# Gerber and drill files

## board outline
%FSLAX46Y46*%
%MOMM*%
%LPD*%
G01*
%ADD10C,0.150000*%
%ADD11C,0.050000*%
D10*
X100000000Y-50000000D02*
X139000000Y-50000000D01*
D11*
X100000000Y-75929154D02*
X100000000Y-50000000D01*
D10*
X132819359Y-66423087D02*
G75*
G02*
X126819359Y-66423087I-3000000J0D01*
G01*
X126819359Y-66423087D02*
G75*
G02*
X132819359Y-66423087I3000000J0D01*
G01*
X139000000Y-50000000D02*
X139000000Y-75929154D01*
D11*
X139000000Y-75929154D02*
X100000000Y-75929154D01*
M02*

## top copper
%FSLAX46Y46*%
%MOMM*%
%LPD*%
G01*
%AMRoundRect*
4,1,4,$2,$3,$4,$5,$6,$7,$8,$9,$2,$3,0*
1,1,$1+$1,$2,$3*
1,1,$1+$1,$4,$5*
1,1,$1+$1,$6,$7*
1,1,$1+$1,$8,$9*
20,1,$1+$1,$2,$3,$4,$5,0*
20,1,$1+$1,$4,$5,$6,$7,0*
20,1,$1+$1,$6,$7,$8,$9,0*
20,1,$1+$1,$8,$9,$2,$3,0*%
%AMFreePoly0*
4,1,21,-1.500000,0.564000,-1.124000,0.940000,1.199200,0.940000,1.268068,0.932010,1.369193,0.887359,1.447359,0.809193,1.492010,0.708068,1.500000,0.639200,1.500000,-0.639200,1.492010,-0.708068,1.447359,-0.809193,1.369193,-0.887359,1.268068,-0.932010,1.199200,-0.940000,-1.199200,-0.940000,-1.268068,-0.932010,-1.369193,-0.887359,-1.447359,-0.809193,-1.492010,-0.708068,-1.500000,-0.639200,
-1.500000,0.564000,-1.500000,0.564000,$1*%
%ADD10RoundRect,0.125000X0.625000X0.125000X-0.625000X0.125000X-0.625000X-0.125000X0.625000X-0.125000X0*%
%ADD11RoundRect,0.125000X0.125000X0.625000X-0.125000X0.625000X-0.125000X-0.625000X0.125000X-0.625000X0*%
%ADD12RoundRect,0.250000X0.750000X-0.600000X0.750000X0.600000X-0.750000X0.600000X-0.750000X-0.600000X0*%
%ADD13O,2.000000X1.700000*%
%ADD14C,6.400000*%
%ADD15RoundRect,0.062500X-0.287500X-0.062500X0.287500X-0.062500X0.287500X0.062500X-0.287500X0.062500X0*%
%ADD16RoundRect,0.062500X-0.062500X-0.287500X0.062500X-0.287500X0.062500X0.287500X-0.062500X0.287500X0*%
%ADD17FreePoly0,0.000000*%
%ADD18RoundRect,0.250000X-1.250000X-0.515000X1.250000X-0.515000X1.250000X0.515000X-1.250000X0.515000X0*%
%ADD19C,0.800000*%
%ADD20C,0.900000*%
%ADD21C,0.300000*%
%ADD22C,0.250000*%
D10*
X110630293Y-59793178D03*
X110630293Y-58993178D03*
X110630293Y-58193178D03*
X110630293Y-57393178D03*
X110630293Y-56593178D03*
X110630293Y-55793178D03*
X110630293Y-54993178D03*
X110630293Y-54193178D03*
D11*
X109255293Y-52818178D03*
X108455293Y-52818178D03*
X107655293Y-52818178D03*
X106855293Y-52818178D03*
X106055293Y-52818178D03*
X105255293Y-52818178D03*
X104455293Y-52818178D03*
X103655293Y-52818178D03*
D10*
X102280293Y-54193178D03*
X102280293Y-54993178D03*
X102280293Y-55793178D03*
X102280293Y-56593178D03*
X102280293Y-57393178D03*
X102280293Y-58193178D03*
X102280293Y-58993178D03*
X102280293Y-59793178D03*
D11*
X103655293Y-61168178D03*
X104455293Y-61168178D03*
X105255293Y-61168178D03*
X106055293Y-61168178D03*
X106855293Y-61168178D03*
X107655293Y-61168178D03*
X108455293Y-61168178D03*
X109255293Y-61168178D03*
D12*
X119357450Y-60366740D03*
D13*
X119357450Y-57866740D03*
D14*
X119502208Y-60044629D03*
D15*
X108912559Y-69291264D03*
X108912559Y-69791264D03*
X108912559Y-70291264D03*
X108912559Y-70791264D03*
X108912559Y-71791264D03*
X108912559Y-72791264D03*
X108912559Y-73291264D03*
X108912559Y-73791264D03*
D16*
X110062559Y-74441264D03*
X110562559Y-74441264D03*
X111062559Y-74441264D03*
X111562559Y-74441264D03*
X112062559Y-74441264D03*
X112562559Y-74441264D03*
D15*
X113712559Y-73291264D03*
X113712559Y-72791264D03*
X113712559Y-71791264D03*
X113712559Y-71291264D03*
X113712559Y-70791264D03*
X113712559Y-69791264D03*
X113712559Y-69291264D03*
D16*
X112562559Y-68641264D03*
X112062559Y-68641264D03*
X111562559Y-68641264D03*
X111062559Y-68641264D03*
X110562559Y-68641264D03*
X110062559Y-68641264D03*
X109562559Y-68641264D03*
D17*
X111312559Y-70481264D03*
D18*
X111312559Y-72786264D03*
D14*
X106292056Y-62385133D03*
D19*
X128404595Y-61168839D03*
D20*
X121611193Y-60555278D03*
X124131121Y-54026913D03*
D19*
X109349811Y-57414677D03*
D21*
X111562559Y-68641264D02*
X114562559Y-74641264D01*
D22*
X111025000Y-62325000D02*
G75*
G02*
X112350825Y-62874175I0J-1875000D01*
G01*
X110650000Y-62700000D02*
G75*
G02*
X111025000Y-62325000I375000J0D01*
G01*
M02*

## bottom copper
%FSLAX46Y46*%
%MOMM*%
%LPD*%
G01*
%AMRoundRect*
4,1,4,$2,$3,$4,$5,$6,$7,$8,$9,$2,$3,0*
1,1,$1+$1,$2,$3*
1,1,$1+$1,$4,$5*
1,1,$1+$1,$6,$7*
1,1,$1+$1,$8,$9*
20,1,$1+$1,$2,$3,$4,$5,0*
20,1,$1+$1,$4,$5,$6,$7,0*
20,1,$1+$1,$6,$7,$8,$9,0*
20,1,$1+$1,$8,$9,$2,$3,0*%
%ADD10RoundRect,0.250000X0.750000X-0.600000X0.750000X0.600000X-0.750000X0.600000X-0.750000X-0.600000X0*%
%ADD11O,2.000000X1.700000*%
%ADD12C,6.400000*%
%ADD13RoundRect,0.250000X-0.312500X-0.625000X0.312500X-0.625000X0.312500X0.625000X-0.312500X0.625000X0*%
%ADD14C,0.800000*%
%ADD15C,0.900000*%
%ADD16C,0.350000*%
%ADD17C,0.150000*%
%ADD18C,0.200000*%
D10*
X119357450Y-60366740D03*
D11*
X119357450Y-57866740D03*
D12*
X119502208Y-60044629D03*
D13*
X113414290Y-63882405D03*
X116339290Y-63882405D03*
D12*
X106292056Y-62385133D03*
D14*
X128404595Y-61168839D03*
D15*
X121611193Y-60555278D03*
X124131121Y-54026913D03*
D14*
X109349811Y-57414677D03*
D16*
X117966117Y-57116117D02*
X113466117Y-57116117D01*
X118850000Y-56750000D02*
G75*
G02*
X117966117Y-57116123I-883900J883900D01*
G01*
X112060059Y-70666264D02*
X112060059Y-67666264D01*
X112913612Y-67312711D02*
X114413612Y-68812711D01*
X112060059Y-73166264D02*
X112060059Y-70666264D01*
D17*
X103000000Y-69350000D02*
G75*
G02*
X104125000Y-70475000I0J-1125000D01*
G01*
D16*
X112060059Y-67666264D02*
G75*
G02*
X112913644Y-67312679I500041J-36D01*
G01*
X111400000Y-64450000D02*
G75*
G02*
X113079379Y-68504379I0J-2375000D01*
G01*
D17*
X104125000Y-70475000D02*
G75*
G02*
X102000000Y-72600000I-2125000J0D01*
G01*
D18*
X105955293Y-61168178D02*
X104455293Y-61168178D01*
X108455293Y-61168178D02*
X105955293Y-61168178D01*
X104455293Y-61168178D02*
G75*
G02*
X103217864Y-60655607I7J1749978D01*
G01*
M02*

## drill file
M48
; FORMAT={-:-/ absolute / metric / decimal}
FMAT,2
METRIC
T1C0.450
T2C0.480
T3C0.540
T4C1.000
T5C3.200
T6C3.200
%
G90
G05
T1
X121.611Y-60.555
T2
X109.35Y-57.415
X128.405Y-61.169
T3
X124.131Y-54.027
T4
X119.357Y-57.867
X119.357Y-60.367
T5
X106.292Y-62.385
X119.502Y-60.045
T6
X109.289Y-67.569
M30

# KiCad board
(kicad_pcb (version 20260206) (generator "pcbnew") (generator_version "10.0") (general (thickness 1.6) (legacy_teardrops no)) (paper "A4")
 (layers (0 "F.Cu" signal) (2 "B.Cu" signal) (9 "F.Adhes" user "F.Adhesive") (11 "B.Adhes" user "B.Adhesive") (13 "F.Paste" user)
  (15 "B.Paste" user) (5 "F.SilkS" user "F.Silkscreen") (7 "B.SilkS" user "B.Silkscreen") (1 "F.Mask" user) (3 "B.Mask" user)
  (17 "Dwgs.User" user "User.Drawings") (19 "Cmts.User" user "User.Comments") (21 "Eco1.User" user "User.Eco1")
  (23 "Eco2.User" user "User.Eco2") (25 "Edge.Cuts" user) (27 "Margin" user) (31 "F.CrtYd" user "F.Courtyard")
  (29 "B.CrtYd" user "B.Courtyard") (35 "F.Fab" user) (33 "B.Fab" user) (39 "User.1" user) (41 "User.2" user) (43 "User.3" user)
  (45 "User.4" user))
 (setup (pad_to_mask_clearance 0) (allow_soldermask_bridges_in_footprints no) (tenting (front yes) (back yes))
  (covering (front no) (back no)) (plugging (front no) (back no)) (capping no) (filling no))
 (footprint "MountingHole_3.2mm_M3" (layer "F.Cu") (at 109.289246 67.568769)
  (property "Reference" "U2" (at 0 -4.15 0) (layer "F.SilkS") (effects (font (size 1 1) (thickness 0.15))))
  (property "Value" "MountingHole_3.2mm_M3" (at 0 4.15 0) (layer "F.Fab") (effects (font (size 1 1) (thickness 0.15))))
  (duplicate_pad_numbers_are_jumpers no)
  (pad "" np_thru_hole circle (at 0 0) (size 3.2 3.2) (drill 3.2) (layers "*.Cu" "*.Mask")))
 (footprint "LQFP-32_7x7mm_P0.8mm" (layer "F.Cu") (at 106.455293 56.993178 180)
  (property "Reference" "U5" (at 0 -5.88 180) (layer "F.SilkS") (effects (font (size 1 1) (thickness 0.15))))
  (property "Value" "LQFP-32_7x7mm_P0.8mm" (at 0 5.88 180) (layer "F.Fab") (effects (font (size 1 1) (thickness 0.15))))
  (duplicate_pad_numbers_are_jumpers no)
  (pad "1" smd roundrect (at -4.175 -2.8 180) (size 1.5 0.5) (layers "F.Cu" "F.Mask" "F.Paste") (roundrect_rratio 0.25) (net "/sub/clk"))
  (pad "2" smd roundrect (at -4.175 -2 180) (size 1.5 0.5) (layers "F.Cu" "F.Mask" "F.Paste") (roundrect_rratio 0.25) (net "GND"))
  (pad "3" smd roundrect (at -4.175 -1.2 180) (size 1.5 0.5) (layers "F.Cu" "F.Mask" "F.Paste") (roundrect_rratio 0.25) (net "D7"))
  (pad "4" smd roundrect (at -4.175 -0.4 180) (size 1.5 0.5) (layers "F.Cu" "F.Mask" "F.Paste") (roundrect_rratio 0.25) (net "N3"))
  (pad "5" smd roundrect (at -4.175 0.4 180) (size 1.5 0.5) (layers "F.Cu" "F.Mask" "F.Paste") (roundrect_rratio 0.25))
  (pad "6" smd roundrect (at -4.175 1.2 180) (size 1.5 0.5) (layers "F.Cu" "F.Mask" "F.Paste") (roundrect_rratio 0.25) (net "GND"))
  (pad "7" smd roundrect (at -4.175 2 180) (size 1.5 0.5) (layers "F.Cu" "F.Mask" "F.Paste") (roundrect_rratio 0.25))
  (pad "8" smd roundrect (at -4.175 2.8 180) (size 1.5 0.5) (layers "F.Cu" "F.Mask" "F.Paste") (roundrect_rratio 0.25) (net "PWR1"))
  (pad "9" smd roundrect (at -2.8 4.175 180) (size 0.5 1.5) (layers "F.Cu" "F.Mask" "F.Paste") (roundrect_rratio 0.25) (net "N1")
   (clearance 0.35))
  (pad "10" smd roundrect (at -2 4.175 180) (size 0.5 1.5) (layers "F.Cu" "F.Mask" "F.Paste") (roundrect_rratio 0.25) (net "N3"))
  (pad "11" smd roundrect (at -1.2 4.175 180) (size 0.5 1.5) (layers "F.Cu" "F.Mask" "F.Paste") (roundrect_rratio 0.25) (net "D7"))
  (pad "12" smd roundrect (at -0.4 4.175 180) (size 0.5 1.5) (layers "F.Cu" "F.Mask" "F.Paste") (roundrect_rratio 0.25) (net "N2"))
  (pad "13" smd roundrect (at 0.4 4.175 180) (size 0.5 1.5) (layers "F.Cu" "F.Mask" "F.Paste") (roundrect_rratio 0.25) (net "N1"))
  (pad "14" smd roundrect (at 1.2 4.175 180) (size 0.5 1.5) (layers "F.Cu" "F.Mask" "F.Paste") (roundrect_rratio 0.25) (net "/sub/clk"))
  (pad "15" smd roundrect (at 2 4.175 180) (size 0.5 1.5) (layers "F.Cu" "F.Mask" "F.Paste") (roundrect_rratio 0.25))
  (pad "16" smd roundrect (at 2.8 4.175 180) (size 0.5 1.5) (layers "F.Cu" "F.Mask" "F.Paste") (roundrect_rratio 0.25))
  (pad "17" smd roundrect (at 4.175 2.8 180) (size 1.5 0.5) (layers "F.Cu" "F.Mask" "F.Paste") (roundrect_rratio 0.25) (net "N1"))
  (pad "18" smd roundrect (at 4.175 2 180) (size 1.5 0.5) (layers "F.Cu" "F.Mask" "F.Paste") (roundrect_rratio 0.25) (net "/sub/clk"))
  (pad "19" smd roundrect (at 4.175 1.2 180) (size 1.5 0.5) (layers "F.Cu" "F.Mask" "F.Paste") (roundrect_rratio 0.25) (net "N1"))
  (pad "20" smd roundrect (at 4.175 0.4 180) (size 1.5 0.5) (layers "F.Cu" "F.Mask" "F.Paste") (roundrect_rratio 0.25) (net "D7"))
  (pad "21" smd roundrect (at 4.175 -0.4 180) (size 1.5 0.5) (layers "F.Cu" "F.Mask" "F.Paste") (roundrect_rratio 0.25) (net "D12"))
  (pad "22" smd roundrect (at 4.175 -1.2 180) (size 1.5 0.5) (layers "F.Cu" "F.Mask" "F.Paste") (roundrect_rratio 0.25))
  (pad "23" smd roundrect (at 4.175 -2 180) (size 1.5 0.5) (layers "F.Cu" "F.Mask" "F.Paste") (roundrect_rratio 0.25))
  (pad "24" smd roundrect (at 4.175 -2.8 180) (size 1.5 0.5) (layers "F.Cu" "F.Mask" "F.Paste") (roundrect_rratio 0.25))
  (pad "25" smd roundrect (at 2.8 -4.175 180) (size 0.5 1.5) (layers "F.Cu" "F.Mask" "F.Paste") (roundrect_rratio 0.25) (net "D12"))
  (pad "26" smd roundrect (at 2 -4.175 180) (size 0.5 1.5) (layers "F.Cu" "F.Mask" "F.Paste") (roundrect_rratio 0.25) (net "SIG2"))
  (pad "27" smd roundrect (at 1.2 -4.175 180) (size 0.5 1.5) (layers "F.Cu" "F.Mask" "F.Paste") (roundrect_rratio 0.25) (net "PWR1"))
  (pad "28" smd roundrect (at 0.4 -4.175 180) (size 0.5 1.5) (layers "F.Cu" "F.Mask" "F.Paste") (roundrect_rratio 0.25) (clearance 0.35))
  (pad "29" smd roundrect (at -0.4 -4.175 180) (size 0.5 1.5) (layers "F.Cu" "F.Mask" "F.Paste") (roundrect_rratio 0.25) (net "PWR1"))
  (pad "30" smd roundrect (at -1.2 -4.175 180) (size 0.5 1.5) (layers "F.Cu" "F.Mask" "F.Paste") (roundrect_rratio 0.25) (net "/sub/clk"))
  (pad "31" smd roundrect (at -2 -4.175 180) (size 0.5 1.5) (layers "F.Cu" "F.Mask" "F.Paste") (roundrect_rratio 0.25) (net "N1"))
  (pad "32" smd roundrect (at -2.8 -4.175 180) (size 0.5 1.5) (layers "F.Cu" "F.Mask" "F.Paste") (roundrect_rratio 0.25) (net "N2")))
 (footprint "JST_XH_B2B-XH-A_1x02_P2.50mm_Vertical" (layer "F.Cu") (at 119.35745 60.36674 90)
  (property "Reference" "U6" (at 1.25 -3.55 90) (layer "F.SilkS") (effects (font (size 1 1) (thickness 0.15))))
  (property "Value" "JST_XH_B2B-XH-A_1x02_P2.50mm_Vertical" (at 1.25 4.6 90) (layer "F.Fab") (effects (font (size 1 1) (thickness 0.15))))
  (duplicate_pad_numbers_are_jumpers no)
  (pad "1" thru_hole roundrect (at 0 0 90) (size 1.7 2) (drill 1) (layers "*.Cu" "*.Mask") (remove_unused_layers no)
   (roundrect_rratio 0.147059) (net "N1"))
  (pad "2" thru_hole oval (at 2.5 0 90) (size 1.7 2) (drill 1) (layers "*.Cu" "*.Mask") (remove_unused_layers no)))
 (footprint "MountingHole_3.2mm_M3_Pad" (layer "F.Cu") (at 119.502208 60.044629)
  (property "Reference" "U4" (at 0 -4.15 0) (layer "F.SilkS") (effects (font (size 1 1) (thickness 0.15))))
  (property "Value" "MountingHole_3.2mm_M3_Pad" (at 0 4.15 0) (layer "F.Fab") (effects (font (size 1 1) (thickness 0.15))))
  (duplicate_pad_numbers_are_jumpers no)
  (pad "1" thru_hole circle (at 0 0) (size 6.4 6.4) (drill 3.2) (layers "*.Cu" "*.Mask") (remove_unused_layers no) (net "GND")
   (zone_connect 2)))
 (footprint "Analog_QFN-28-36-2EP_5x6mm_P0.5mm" (layer "F.Cu") (at 111.312559 71.541264)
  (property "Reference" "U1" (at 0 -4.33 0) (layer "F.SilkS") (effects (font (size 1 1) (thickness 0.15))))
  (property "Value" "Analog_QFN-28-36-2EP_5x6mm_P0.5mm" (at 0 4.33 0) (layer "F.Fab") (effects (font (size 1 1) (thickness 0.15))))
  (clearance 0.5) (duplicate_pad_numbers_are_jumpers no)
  (pad "" smd roundrect (at -0.75 -1.53) (size 1.21 0.76) (layers "F.Paste") (roundrect_rratio 0.25) (chamfer_ratio 0.4) (chamfer top_left)
   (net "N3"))
  (pad "" smd roundrect (at -0.75 -0.59) (size 1.21 0.76) (layers "F.Paste") (roundrect_rratio 0.25) (clearance 0.1))
  (pad "" smd roundrect (at -0.7475 0.875) (size 1.205 0.55) (layers "F.Paste") (roundrect_rratio 0.25) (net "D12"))
  (pad "" smd roundrect (at -0.7475 1.625) (size 1.205 0.55) (layers "F.Paste") (roundrect_rratio 0.25) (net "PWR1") (clearance 0.35))
  (pad "" smd roundrect (at 0.7475 0.875) (size 1.205 0.55) (layers "F.Paste") (roundrect_rratio 0.25) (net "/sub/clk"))
  (pad "" smd roundrect (at 0.7475 1.625) (size 1.205 0.55) (layers "F.Paste") (roundrect_rratio 0.25) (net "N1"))
  (pad "" smd roundrect (at 0.75 -1.53) (size 1.21 0.76) (layers "F.Paste") (roundrect_rratio 0.25) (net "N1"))
  (pad "" smd roundrect (at 0.75 -0.59) (size 1.21 0.76) (layers "F.Paste") (roundrect_rratio 0.25) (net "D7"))
  (pad "1" smd roundrect (at -2.4 -2.25) (size 0.7 0.25) (layers "F.Cu" "F.Mask" "F.Paste") (roundrect_rratio 0.25) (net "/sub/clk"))
  (pad "2" smd roundrect (at -2.4 -1.75) (size 0.7 0.25) (layers "F.Cu" "F.Mask" "F.Paste") (roundrect_rratio 0.25) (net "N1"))
  (pad "3" smd roundrect (at -2.4 -1.25) (size 0.7 0.25) (layers "F.Cu" "F.Mask" "F.Paste") (roundrect_rratio 0.25))
  (pad "4" smd roundrect (at -2.4 -0.75) (size 0.7 0.25) (layers "F.Cu" "F.Mask" "F.Paste") (roundrect_rratio 0.25))
  (pad "6" smd roundrect (at -2.4 0.25) (size 0.7 0.25) (layers "F.Cu" "F.Mask" "F.Paste") (roundrect_rratio 0.25) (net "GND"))
  (pad "8" smd roundrect (at -2.4 1.25) (size 0.7 0.25) (layers "F.Cu" "F.Mask" "F.Paste") (roundrect_rratio 0.25))
  (pad "9" smd roundrect (at -2.4 1.75) (size 0.7 0.25) (layers "F.Cu" "F.Mask" "F.Paste") (roundrect_rratio 0.25) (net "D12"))
  (pad "10" smd roundrect (at -2.4 2.25) (size 0.7 0.25) (layers "F.Cu" "F.Mask" "F.Paste") (roundrect_rratio 0.25) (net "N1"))
  (pad "12" smd roundrect (at -1.25 2.9) (size 0.25 0.7) (layers "F.Cu" "F.Mask" "F.Paste") (roundrect_rratio 0.25))
  (pad "13" smd roundrect (at -0.75 2.9) (size 0.25 0.7) (layers "F.Cu" "F.Mask" "F.Paste") (roundrect_rratio 0.25) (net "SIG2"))
  (pad "14" smd roundrect (at -0.25 2.9) (size 0.25 0.7) (layers "F.Cu" "F.Mask" "F.Paste") (roundrect_rratio 0.25) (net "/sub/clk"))
  (pad "15" smd roundrect (at 0.25 2.9) (size 0.25 0.7) (layers "F.Cu" "F.Mask" "F.Paste") (roundrect_rratio 0.25))
  (pad "16" smd roundrect (at 0.75 2.9) (size 0.25 0.7) (layers "F.Cu" "F.Mask" "F.Paste") (roundrect_rratio 0.25) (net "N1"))
  (pad "17" smd roundrect (at 1.25 2.9) (size 0.25 0.7) (layers "F.Cu" "F.Mask" "F.Paste") (roundrect_rratio 0.25) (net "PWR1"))
  (pad "20" smd roundrect (at 2.4 1.75) (size 0.7 0.25) (layers "F.Cu" "F.Mask" "F.Paste") (roundrect_rratio 0.25) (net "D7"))
  (pad "21" smd roundrect (at 2.4 1.25) (size 0.7 0.25) (layers "F.Cu" "F.Mask" "F.Paste") (roundrect_rratio 0.25) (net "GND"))
  (pad "23" smd roundrect (at 2.4 0.25) (size 0.7 0.25) (layers "F.Cu" "F.Mask" "F.Paste") (roundrect_rratio 0.25))
  (pad "24" smd roundrect (at 2.4 -0.25) (size 0.7 0.25) (layers "F.Cu" "F.Mask" "F.Paste") (roundrect_rratio 0.25) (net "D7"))
  (pad "25" smd roundrect (at 2.4 -0.75) (size 0.7 0.25) (layers "F.Cu" "F.Mask" "F.Paste") (roundrect_rratio 0.25) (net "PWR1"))
  (pad "27" smd roundrect (at 2.4 -1.75) (size 0.7 0.25) (layers "F.Cu" "F.Mask" "F.Paste") (roundrect_rratio 0.25) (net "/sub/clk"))
  (pad "28" smd roundrect (at 2.4 -2.25) (size 0.7 0.25) (layers "F.Cu" "F.Mask" "F.Paste") (roundrect_rratio 0.25) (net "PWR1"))
  (pad "30" smd roundrect (at 1.25 -2.9) (size 0.25 0.7) (layers "F.Cu" "F.Mask" "F.Paste") (roundrect_rratio 0.25))
  (pad "31" smd roundrect (at 0.75 -2.9) (size 0.25 0.7) (layers "F.Cu" "F.Mask" "F.Paste") (roundrect_rratio 0.25))
  (pad "32" smd roundrect (at 0.25 -2.9) (size 0.25 0.7) (layers "F.Cu" "F.Mask" "F.Paste") (roundrect_rratio 0.25))
  (pad "33" smd roundrect (at -0.25 -2.9) (size 0.25 0.7) (layers "F.Cu" "F.Mask" "F.Paste") (roundrect_rratio 0.25) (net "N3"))
  (pad "34" smd roundrect (at -0.75 -2.9) (size 0.25 0.7) (layers "F.Cu" "F.Mask" "F.Paste") (roundrect_rratio 0.25))
  (pad "35" smd roundrect (at -1.25 -2.9) (size 0.25 0.7) (layers "F.Cu" "F.Mask" "F.Paste") (roundrect_rratio 0.25))
  (pad "36" smd roundrect (at -1.75 -2.9) (size 0.25 0.7) (layers "F.Cu" "F.Mask" "F.Paste") (roundrect_rratio 0.25) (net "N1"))
  (pad "37" smd roundrect (at 0 -1.06) (size 3 1.88) (layers "F.Cu" "F.Mask") (roundrect_rratio 0.16) (chamfer_ratio 0.2) (chamfer top_left)
   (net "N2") (zone_connect 2))
  (pad "38" smd roundrect (at 0 1.245) (size 3 1.53) (layers "F.Cu" "F.Mask") (roundrect_rratio 0.1633986928) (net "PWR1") (zone_connect 2)))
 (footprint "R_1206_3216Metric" (layer "B.Cu") (at 114.87679 63.882405)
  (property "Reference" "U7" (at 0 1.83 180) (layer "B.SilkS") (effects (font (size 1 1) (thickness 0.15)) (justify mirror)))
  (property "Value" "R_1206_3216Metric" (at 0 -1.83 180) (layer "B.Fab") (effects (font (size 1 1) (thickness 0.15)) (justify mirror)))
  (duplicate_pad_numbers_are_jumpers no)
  (pad "1" smd roundrect (at -1.4625 0) (size 1.125 1.75) (layers "B.Cu" "B.Mask" "B.Paste") (roundrect_rratio 0.222222) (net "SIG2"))
  (pad "2" smd roundrect (at 1.4625 0) (size 1.125 1.75) (layers "B.Cu" "B.Mask" "B.Paste") (roundrect_rratio 0.222222) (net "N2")))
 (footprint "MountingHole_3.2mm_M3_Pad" (layer "B.Cu") (at 106.292056 62.385133 90)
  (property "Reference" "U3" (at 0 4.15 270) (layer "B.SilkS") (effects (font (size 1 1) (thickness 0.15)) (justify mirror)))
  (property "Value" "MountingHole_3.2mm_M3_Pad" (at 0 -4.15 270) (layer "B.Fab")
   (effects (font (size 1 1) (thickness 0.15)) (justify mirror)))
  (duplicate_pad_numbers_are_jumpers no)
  (pad "1" thru_hole circle (at 0 0 90) (size 6.4 6.4) (drill 3.2) (layers "*.Cu" "*.Mask") (remove_unused_layers no) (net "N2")
   (clearance 0.1) (zone_connect 2)))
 (gr_line (start 100 50) (end 139 50) (stroke (width 0.15) (type default)) (layer "Edge.Cuts"))
 (gr_line (start 100 75.929154) (end 100 50) (stroke (width 0.05) (type default)) (layer "Edge.Cuts"))
 (gr_circle (center 129.819359 66.423087) (end 132.819359 66.423087) (stroke (width 0.15) (type default)) (fill no) (layer "Edge.Cuts"))
 (gr_line (start 139 50) (end 139 75.929154) (stroke (width 0.15) (type default)) (layer "Edge.Cuts"))
 (gr_line (start 139 75.929154) (end 100 75.929154) (stroke (width 0.05) (type default)) (layer "Edge.Cuts"))
 (segment (start 111.562559 68.641264) (end 114.562559 74.641264) (width 0.3) (layer "F.Cu") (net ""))
 (arc (start 111.025 62.325) (mid 111.742531 62.467726) (end 112.350825 62.874175) (width 0.25) (locked yes) (layer "F.Cu") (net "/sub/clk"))
 (arc (start 110.65 62.7) (mid 110.759835 62.434835) (end 111.025 62.325) (width 0.25) (layer "F.Cu") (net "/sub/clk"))
 (via (at 128.404595 61.168839) (size 0.8) (drill 0.48) (layers "F.Cu" "B.Cu") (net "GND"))
 (via (at 121.611193 60.555278) (size 0.9) (drill 0.45) (layers "F.Cu" "B.Cu") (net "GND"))
 (segment (start 117.966117 57.116117) (end 113.466117 57.116117) (width 0.35) (layer "B.Cu") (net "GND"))
 (arc (start 118.85 56.75) (mid 118.444471 57.020966) (end 117.966117 57.116117) (width 0.35) (layer "B.Cu") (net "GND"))
 (via (at 124.131121 54.026913) (size 0.9) (drill 0.54) (layers "F.Cu" "B.Cu") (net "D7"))
 (via (at 109.349811 57.414677) (size 0.8) (drill 0.48) (layers "F.Cu" "B.Cu") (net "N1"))
 (segment (start 112.060059 70.666264) (end 112.060059 67.666264) (width 0.35) (layer "B.Cu") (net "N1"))
 (segment (start 112.913612 67.312711) (end 114.413612 68.812711) (width 0.35) (layer "B.Cu") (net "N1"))
 (segment (start 112.060059 73.166264) (end 112.060059 70.666264) (width 0.35) (layer "B.Cu") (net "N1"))
 (arc (start 103 69.35) (mid 103.795495 69.679505) (end 104.125 70.475) (width 0.15) (layer "B.Cu") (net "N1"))
 (arc (start 112.060059 67.666264) (mid 112.368717 67.204324) (end 112.913612 67.312711) (width 0.35) (layer "B.Cu") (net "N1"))
 (arc (start 111.4 64.45) (mid 113.594214 65.916127) (end 113.079379 68.504379) (width 0.35) (layer "B.Cu") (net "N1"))
 (arc (start 104.125 70.475) (mid 103.502602 71.977602) (end 102 72.6) (width 0.15) (locked yes) (layer "B.Cu") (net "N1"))
 (segment (start 105.955293 61.168178) (end 104.455293 61.168178) (width 0.2) (layer "B.Cu") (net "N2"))
 (segment (start 108.455293 61.168178) (end 105.955293 61.168178) (width 0.2) (layer "B.Cu") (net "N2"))
 (arc (start 104.455293 61.168178) (mid 103.785597 61.034967) (end 103.217856 60.655615) (width 0.2) (layer "B.Cu") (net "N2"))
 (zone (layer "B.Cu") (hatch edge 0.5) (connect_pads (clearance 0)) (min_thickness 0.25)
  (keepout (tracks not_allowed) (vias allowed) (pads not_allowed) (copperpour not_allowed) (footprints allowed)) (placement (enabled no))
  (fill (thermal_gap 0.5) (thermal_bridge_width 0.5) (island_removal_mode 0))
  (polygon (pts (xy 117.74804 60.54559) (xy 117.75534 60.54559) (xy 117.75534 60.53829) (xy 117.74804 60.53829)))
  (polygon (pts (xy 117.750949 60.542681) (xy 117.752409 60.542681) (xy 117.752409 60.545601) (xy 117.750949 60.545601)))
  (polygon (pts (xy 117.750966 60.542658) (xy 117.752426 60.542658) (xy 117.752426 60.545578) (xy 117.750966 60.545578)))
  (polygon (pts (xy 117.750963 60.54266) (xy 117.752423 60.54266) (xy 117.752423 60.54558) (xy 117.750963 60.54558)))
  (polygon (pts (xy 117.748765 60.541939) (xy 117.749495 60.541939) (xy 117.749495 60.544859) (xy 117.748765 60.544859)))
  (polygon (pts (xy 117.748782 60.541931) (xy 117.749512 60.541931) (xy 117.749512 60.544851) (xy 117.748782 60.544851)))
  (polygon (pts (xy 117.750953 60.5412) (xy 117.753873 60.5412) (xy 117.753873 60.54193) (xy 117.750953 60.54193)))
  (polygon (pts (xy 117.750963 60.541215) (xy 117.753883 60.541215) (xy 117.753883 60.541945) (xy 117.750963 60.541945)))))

